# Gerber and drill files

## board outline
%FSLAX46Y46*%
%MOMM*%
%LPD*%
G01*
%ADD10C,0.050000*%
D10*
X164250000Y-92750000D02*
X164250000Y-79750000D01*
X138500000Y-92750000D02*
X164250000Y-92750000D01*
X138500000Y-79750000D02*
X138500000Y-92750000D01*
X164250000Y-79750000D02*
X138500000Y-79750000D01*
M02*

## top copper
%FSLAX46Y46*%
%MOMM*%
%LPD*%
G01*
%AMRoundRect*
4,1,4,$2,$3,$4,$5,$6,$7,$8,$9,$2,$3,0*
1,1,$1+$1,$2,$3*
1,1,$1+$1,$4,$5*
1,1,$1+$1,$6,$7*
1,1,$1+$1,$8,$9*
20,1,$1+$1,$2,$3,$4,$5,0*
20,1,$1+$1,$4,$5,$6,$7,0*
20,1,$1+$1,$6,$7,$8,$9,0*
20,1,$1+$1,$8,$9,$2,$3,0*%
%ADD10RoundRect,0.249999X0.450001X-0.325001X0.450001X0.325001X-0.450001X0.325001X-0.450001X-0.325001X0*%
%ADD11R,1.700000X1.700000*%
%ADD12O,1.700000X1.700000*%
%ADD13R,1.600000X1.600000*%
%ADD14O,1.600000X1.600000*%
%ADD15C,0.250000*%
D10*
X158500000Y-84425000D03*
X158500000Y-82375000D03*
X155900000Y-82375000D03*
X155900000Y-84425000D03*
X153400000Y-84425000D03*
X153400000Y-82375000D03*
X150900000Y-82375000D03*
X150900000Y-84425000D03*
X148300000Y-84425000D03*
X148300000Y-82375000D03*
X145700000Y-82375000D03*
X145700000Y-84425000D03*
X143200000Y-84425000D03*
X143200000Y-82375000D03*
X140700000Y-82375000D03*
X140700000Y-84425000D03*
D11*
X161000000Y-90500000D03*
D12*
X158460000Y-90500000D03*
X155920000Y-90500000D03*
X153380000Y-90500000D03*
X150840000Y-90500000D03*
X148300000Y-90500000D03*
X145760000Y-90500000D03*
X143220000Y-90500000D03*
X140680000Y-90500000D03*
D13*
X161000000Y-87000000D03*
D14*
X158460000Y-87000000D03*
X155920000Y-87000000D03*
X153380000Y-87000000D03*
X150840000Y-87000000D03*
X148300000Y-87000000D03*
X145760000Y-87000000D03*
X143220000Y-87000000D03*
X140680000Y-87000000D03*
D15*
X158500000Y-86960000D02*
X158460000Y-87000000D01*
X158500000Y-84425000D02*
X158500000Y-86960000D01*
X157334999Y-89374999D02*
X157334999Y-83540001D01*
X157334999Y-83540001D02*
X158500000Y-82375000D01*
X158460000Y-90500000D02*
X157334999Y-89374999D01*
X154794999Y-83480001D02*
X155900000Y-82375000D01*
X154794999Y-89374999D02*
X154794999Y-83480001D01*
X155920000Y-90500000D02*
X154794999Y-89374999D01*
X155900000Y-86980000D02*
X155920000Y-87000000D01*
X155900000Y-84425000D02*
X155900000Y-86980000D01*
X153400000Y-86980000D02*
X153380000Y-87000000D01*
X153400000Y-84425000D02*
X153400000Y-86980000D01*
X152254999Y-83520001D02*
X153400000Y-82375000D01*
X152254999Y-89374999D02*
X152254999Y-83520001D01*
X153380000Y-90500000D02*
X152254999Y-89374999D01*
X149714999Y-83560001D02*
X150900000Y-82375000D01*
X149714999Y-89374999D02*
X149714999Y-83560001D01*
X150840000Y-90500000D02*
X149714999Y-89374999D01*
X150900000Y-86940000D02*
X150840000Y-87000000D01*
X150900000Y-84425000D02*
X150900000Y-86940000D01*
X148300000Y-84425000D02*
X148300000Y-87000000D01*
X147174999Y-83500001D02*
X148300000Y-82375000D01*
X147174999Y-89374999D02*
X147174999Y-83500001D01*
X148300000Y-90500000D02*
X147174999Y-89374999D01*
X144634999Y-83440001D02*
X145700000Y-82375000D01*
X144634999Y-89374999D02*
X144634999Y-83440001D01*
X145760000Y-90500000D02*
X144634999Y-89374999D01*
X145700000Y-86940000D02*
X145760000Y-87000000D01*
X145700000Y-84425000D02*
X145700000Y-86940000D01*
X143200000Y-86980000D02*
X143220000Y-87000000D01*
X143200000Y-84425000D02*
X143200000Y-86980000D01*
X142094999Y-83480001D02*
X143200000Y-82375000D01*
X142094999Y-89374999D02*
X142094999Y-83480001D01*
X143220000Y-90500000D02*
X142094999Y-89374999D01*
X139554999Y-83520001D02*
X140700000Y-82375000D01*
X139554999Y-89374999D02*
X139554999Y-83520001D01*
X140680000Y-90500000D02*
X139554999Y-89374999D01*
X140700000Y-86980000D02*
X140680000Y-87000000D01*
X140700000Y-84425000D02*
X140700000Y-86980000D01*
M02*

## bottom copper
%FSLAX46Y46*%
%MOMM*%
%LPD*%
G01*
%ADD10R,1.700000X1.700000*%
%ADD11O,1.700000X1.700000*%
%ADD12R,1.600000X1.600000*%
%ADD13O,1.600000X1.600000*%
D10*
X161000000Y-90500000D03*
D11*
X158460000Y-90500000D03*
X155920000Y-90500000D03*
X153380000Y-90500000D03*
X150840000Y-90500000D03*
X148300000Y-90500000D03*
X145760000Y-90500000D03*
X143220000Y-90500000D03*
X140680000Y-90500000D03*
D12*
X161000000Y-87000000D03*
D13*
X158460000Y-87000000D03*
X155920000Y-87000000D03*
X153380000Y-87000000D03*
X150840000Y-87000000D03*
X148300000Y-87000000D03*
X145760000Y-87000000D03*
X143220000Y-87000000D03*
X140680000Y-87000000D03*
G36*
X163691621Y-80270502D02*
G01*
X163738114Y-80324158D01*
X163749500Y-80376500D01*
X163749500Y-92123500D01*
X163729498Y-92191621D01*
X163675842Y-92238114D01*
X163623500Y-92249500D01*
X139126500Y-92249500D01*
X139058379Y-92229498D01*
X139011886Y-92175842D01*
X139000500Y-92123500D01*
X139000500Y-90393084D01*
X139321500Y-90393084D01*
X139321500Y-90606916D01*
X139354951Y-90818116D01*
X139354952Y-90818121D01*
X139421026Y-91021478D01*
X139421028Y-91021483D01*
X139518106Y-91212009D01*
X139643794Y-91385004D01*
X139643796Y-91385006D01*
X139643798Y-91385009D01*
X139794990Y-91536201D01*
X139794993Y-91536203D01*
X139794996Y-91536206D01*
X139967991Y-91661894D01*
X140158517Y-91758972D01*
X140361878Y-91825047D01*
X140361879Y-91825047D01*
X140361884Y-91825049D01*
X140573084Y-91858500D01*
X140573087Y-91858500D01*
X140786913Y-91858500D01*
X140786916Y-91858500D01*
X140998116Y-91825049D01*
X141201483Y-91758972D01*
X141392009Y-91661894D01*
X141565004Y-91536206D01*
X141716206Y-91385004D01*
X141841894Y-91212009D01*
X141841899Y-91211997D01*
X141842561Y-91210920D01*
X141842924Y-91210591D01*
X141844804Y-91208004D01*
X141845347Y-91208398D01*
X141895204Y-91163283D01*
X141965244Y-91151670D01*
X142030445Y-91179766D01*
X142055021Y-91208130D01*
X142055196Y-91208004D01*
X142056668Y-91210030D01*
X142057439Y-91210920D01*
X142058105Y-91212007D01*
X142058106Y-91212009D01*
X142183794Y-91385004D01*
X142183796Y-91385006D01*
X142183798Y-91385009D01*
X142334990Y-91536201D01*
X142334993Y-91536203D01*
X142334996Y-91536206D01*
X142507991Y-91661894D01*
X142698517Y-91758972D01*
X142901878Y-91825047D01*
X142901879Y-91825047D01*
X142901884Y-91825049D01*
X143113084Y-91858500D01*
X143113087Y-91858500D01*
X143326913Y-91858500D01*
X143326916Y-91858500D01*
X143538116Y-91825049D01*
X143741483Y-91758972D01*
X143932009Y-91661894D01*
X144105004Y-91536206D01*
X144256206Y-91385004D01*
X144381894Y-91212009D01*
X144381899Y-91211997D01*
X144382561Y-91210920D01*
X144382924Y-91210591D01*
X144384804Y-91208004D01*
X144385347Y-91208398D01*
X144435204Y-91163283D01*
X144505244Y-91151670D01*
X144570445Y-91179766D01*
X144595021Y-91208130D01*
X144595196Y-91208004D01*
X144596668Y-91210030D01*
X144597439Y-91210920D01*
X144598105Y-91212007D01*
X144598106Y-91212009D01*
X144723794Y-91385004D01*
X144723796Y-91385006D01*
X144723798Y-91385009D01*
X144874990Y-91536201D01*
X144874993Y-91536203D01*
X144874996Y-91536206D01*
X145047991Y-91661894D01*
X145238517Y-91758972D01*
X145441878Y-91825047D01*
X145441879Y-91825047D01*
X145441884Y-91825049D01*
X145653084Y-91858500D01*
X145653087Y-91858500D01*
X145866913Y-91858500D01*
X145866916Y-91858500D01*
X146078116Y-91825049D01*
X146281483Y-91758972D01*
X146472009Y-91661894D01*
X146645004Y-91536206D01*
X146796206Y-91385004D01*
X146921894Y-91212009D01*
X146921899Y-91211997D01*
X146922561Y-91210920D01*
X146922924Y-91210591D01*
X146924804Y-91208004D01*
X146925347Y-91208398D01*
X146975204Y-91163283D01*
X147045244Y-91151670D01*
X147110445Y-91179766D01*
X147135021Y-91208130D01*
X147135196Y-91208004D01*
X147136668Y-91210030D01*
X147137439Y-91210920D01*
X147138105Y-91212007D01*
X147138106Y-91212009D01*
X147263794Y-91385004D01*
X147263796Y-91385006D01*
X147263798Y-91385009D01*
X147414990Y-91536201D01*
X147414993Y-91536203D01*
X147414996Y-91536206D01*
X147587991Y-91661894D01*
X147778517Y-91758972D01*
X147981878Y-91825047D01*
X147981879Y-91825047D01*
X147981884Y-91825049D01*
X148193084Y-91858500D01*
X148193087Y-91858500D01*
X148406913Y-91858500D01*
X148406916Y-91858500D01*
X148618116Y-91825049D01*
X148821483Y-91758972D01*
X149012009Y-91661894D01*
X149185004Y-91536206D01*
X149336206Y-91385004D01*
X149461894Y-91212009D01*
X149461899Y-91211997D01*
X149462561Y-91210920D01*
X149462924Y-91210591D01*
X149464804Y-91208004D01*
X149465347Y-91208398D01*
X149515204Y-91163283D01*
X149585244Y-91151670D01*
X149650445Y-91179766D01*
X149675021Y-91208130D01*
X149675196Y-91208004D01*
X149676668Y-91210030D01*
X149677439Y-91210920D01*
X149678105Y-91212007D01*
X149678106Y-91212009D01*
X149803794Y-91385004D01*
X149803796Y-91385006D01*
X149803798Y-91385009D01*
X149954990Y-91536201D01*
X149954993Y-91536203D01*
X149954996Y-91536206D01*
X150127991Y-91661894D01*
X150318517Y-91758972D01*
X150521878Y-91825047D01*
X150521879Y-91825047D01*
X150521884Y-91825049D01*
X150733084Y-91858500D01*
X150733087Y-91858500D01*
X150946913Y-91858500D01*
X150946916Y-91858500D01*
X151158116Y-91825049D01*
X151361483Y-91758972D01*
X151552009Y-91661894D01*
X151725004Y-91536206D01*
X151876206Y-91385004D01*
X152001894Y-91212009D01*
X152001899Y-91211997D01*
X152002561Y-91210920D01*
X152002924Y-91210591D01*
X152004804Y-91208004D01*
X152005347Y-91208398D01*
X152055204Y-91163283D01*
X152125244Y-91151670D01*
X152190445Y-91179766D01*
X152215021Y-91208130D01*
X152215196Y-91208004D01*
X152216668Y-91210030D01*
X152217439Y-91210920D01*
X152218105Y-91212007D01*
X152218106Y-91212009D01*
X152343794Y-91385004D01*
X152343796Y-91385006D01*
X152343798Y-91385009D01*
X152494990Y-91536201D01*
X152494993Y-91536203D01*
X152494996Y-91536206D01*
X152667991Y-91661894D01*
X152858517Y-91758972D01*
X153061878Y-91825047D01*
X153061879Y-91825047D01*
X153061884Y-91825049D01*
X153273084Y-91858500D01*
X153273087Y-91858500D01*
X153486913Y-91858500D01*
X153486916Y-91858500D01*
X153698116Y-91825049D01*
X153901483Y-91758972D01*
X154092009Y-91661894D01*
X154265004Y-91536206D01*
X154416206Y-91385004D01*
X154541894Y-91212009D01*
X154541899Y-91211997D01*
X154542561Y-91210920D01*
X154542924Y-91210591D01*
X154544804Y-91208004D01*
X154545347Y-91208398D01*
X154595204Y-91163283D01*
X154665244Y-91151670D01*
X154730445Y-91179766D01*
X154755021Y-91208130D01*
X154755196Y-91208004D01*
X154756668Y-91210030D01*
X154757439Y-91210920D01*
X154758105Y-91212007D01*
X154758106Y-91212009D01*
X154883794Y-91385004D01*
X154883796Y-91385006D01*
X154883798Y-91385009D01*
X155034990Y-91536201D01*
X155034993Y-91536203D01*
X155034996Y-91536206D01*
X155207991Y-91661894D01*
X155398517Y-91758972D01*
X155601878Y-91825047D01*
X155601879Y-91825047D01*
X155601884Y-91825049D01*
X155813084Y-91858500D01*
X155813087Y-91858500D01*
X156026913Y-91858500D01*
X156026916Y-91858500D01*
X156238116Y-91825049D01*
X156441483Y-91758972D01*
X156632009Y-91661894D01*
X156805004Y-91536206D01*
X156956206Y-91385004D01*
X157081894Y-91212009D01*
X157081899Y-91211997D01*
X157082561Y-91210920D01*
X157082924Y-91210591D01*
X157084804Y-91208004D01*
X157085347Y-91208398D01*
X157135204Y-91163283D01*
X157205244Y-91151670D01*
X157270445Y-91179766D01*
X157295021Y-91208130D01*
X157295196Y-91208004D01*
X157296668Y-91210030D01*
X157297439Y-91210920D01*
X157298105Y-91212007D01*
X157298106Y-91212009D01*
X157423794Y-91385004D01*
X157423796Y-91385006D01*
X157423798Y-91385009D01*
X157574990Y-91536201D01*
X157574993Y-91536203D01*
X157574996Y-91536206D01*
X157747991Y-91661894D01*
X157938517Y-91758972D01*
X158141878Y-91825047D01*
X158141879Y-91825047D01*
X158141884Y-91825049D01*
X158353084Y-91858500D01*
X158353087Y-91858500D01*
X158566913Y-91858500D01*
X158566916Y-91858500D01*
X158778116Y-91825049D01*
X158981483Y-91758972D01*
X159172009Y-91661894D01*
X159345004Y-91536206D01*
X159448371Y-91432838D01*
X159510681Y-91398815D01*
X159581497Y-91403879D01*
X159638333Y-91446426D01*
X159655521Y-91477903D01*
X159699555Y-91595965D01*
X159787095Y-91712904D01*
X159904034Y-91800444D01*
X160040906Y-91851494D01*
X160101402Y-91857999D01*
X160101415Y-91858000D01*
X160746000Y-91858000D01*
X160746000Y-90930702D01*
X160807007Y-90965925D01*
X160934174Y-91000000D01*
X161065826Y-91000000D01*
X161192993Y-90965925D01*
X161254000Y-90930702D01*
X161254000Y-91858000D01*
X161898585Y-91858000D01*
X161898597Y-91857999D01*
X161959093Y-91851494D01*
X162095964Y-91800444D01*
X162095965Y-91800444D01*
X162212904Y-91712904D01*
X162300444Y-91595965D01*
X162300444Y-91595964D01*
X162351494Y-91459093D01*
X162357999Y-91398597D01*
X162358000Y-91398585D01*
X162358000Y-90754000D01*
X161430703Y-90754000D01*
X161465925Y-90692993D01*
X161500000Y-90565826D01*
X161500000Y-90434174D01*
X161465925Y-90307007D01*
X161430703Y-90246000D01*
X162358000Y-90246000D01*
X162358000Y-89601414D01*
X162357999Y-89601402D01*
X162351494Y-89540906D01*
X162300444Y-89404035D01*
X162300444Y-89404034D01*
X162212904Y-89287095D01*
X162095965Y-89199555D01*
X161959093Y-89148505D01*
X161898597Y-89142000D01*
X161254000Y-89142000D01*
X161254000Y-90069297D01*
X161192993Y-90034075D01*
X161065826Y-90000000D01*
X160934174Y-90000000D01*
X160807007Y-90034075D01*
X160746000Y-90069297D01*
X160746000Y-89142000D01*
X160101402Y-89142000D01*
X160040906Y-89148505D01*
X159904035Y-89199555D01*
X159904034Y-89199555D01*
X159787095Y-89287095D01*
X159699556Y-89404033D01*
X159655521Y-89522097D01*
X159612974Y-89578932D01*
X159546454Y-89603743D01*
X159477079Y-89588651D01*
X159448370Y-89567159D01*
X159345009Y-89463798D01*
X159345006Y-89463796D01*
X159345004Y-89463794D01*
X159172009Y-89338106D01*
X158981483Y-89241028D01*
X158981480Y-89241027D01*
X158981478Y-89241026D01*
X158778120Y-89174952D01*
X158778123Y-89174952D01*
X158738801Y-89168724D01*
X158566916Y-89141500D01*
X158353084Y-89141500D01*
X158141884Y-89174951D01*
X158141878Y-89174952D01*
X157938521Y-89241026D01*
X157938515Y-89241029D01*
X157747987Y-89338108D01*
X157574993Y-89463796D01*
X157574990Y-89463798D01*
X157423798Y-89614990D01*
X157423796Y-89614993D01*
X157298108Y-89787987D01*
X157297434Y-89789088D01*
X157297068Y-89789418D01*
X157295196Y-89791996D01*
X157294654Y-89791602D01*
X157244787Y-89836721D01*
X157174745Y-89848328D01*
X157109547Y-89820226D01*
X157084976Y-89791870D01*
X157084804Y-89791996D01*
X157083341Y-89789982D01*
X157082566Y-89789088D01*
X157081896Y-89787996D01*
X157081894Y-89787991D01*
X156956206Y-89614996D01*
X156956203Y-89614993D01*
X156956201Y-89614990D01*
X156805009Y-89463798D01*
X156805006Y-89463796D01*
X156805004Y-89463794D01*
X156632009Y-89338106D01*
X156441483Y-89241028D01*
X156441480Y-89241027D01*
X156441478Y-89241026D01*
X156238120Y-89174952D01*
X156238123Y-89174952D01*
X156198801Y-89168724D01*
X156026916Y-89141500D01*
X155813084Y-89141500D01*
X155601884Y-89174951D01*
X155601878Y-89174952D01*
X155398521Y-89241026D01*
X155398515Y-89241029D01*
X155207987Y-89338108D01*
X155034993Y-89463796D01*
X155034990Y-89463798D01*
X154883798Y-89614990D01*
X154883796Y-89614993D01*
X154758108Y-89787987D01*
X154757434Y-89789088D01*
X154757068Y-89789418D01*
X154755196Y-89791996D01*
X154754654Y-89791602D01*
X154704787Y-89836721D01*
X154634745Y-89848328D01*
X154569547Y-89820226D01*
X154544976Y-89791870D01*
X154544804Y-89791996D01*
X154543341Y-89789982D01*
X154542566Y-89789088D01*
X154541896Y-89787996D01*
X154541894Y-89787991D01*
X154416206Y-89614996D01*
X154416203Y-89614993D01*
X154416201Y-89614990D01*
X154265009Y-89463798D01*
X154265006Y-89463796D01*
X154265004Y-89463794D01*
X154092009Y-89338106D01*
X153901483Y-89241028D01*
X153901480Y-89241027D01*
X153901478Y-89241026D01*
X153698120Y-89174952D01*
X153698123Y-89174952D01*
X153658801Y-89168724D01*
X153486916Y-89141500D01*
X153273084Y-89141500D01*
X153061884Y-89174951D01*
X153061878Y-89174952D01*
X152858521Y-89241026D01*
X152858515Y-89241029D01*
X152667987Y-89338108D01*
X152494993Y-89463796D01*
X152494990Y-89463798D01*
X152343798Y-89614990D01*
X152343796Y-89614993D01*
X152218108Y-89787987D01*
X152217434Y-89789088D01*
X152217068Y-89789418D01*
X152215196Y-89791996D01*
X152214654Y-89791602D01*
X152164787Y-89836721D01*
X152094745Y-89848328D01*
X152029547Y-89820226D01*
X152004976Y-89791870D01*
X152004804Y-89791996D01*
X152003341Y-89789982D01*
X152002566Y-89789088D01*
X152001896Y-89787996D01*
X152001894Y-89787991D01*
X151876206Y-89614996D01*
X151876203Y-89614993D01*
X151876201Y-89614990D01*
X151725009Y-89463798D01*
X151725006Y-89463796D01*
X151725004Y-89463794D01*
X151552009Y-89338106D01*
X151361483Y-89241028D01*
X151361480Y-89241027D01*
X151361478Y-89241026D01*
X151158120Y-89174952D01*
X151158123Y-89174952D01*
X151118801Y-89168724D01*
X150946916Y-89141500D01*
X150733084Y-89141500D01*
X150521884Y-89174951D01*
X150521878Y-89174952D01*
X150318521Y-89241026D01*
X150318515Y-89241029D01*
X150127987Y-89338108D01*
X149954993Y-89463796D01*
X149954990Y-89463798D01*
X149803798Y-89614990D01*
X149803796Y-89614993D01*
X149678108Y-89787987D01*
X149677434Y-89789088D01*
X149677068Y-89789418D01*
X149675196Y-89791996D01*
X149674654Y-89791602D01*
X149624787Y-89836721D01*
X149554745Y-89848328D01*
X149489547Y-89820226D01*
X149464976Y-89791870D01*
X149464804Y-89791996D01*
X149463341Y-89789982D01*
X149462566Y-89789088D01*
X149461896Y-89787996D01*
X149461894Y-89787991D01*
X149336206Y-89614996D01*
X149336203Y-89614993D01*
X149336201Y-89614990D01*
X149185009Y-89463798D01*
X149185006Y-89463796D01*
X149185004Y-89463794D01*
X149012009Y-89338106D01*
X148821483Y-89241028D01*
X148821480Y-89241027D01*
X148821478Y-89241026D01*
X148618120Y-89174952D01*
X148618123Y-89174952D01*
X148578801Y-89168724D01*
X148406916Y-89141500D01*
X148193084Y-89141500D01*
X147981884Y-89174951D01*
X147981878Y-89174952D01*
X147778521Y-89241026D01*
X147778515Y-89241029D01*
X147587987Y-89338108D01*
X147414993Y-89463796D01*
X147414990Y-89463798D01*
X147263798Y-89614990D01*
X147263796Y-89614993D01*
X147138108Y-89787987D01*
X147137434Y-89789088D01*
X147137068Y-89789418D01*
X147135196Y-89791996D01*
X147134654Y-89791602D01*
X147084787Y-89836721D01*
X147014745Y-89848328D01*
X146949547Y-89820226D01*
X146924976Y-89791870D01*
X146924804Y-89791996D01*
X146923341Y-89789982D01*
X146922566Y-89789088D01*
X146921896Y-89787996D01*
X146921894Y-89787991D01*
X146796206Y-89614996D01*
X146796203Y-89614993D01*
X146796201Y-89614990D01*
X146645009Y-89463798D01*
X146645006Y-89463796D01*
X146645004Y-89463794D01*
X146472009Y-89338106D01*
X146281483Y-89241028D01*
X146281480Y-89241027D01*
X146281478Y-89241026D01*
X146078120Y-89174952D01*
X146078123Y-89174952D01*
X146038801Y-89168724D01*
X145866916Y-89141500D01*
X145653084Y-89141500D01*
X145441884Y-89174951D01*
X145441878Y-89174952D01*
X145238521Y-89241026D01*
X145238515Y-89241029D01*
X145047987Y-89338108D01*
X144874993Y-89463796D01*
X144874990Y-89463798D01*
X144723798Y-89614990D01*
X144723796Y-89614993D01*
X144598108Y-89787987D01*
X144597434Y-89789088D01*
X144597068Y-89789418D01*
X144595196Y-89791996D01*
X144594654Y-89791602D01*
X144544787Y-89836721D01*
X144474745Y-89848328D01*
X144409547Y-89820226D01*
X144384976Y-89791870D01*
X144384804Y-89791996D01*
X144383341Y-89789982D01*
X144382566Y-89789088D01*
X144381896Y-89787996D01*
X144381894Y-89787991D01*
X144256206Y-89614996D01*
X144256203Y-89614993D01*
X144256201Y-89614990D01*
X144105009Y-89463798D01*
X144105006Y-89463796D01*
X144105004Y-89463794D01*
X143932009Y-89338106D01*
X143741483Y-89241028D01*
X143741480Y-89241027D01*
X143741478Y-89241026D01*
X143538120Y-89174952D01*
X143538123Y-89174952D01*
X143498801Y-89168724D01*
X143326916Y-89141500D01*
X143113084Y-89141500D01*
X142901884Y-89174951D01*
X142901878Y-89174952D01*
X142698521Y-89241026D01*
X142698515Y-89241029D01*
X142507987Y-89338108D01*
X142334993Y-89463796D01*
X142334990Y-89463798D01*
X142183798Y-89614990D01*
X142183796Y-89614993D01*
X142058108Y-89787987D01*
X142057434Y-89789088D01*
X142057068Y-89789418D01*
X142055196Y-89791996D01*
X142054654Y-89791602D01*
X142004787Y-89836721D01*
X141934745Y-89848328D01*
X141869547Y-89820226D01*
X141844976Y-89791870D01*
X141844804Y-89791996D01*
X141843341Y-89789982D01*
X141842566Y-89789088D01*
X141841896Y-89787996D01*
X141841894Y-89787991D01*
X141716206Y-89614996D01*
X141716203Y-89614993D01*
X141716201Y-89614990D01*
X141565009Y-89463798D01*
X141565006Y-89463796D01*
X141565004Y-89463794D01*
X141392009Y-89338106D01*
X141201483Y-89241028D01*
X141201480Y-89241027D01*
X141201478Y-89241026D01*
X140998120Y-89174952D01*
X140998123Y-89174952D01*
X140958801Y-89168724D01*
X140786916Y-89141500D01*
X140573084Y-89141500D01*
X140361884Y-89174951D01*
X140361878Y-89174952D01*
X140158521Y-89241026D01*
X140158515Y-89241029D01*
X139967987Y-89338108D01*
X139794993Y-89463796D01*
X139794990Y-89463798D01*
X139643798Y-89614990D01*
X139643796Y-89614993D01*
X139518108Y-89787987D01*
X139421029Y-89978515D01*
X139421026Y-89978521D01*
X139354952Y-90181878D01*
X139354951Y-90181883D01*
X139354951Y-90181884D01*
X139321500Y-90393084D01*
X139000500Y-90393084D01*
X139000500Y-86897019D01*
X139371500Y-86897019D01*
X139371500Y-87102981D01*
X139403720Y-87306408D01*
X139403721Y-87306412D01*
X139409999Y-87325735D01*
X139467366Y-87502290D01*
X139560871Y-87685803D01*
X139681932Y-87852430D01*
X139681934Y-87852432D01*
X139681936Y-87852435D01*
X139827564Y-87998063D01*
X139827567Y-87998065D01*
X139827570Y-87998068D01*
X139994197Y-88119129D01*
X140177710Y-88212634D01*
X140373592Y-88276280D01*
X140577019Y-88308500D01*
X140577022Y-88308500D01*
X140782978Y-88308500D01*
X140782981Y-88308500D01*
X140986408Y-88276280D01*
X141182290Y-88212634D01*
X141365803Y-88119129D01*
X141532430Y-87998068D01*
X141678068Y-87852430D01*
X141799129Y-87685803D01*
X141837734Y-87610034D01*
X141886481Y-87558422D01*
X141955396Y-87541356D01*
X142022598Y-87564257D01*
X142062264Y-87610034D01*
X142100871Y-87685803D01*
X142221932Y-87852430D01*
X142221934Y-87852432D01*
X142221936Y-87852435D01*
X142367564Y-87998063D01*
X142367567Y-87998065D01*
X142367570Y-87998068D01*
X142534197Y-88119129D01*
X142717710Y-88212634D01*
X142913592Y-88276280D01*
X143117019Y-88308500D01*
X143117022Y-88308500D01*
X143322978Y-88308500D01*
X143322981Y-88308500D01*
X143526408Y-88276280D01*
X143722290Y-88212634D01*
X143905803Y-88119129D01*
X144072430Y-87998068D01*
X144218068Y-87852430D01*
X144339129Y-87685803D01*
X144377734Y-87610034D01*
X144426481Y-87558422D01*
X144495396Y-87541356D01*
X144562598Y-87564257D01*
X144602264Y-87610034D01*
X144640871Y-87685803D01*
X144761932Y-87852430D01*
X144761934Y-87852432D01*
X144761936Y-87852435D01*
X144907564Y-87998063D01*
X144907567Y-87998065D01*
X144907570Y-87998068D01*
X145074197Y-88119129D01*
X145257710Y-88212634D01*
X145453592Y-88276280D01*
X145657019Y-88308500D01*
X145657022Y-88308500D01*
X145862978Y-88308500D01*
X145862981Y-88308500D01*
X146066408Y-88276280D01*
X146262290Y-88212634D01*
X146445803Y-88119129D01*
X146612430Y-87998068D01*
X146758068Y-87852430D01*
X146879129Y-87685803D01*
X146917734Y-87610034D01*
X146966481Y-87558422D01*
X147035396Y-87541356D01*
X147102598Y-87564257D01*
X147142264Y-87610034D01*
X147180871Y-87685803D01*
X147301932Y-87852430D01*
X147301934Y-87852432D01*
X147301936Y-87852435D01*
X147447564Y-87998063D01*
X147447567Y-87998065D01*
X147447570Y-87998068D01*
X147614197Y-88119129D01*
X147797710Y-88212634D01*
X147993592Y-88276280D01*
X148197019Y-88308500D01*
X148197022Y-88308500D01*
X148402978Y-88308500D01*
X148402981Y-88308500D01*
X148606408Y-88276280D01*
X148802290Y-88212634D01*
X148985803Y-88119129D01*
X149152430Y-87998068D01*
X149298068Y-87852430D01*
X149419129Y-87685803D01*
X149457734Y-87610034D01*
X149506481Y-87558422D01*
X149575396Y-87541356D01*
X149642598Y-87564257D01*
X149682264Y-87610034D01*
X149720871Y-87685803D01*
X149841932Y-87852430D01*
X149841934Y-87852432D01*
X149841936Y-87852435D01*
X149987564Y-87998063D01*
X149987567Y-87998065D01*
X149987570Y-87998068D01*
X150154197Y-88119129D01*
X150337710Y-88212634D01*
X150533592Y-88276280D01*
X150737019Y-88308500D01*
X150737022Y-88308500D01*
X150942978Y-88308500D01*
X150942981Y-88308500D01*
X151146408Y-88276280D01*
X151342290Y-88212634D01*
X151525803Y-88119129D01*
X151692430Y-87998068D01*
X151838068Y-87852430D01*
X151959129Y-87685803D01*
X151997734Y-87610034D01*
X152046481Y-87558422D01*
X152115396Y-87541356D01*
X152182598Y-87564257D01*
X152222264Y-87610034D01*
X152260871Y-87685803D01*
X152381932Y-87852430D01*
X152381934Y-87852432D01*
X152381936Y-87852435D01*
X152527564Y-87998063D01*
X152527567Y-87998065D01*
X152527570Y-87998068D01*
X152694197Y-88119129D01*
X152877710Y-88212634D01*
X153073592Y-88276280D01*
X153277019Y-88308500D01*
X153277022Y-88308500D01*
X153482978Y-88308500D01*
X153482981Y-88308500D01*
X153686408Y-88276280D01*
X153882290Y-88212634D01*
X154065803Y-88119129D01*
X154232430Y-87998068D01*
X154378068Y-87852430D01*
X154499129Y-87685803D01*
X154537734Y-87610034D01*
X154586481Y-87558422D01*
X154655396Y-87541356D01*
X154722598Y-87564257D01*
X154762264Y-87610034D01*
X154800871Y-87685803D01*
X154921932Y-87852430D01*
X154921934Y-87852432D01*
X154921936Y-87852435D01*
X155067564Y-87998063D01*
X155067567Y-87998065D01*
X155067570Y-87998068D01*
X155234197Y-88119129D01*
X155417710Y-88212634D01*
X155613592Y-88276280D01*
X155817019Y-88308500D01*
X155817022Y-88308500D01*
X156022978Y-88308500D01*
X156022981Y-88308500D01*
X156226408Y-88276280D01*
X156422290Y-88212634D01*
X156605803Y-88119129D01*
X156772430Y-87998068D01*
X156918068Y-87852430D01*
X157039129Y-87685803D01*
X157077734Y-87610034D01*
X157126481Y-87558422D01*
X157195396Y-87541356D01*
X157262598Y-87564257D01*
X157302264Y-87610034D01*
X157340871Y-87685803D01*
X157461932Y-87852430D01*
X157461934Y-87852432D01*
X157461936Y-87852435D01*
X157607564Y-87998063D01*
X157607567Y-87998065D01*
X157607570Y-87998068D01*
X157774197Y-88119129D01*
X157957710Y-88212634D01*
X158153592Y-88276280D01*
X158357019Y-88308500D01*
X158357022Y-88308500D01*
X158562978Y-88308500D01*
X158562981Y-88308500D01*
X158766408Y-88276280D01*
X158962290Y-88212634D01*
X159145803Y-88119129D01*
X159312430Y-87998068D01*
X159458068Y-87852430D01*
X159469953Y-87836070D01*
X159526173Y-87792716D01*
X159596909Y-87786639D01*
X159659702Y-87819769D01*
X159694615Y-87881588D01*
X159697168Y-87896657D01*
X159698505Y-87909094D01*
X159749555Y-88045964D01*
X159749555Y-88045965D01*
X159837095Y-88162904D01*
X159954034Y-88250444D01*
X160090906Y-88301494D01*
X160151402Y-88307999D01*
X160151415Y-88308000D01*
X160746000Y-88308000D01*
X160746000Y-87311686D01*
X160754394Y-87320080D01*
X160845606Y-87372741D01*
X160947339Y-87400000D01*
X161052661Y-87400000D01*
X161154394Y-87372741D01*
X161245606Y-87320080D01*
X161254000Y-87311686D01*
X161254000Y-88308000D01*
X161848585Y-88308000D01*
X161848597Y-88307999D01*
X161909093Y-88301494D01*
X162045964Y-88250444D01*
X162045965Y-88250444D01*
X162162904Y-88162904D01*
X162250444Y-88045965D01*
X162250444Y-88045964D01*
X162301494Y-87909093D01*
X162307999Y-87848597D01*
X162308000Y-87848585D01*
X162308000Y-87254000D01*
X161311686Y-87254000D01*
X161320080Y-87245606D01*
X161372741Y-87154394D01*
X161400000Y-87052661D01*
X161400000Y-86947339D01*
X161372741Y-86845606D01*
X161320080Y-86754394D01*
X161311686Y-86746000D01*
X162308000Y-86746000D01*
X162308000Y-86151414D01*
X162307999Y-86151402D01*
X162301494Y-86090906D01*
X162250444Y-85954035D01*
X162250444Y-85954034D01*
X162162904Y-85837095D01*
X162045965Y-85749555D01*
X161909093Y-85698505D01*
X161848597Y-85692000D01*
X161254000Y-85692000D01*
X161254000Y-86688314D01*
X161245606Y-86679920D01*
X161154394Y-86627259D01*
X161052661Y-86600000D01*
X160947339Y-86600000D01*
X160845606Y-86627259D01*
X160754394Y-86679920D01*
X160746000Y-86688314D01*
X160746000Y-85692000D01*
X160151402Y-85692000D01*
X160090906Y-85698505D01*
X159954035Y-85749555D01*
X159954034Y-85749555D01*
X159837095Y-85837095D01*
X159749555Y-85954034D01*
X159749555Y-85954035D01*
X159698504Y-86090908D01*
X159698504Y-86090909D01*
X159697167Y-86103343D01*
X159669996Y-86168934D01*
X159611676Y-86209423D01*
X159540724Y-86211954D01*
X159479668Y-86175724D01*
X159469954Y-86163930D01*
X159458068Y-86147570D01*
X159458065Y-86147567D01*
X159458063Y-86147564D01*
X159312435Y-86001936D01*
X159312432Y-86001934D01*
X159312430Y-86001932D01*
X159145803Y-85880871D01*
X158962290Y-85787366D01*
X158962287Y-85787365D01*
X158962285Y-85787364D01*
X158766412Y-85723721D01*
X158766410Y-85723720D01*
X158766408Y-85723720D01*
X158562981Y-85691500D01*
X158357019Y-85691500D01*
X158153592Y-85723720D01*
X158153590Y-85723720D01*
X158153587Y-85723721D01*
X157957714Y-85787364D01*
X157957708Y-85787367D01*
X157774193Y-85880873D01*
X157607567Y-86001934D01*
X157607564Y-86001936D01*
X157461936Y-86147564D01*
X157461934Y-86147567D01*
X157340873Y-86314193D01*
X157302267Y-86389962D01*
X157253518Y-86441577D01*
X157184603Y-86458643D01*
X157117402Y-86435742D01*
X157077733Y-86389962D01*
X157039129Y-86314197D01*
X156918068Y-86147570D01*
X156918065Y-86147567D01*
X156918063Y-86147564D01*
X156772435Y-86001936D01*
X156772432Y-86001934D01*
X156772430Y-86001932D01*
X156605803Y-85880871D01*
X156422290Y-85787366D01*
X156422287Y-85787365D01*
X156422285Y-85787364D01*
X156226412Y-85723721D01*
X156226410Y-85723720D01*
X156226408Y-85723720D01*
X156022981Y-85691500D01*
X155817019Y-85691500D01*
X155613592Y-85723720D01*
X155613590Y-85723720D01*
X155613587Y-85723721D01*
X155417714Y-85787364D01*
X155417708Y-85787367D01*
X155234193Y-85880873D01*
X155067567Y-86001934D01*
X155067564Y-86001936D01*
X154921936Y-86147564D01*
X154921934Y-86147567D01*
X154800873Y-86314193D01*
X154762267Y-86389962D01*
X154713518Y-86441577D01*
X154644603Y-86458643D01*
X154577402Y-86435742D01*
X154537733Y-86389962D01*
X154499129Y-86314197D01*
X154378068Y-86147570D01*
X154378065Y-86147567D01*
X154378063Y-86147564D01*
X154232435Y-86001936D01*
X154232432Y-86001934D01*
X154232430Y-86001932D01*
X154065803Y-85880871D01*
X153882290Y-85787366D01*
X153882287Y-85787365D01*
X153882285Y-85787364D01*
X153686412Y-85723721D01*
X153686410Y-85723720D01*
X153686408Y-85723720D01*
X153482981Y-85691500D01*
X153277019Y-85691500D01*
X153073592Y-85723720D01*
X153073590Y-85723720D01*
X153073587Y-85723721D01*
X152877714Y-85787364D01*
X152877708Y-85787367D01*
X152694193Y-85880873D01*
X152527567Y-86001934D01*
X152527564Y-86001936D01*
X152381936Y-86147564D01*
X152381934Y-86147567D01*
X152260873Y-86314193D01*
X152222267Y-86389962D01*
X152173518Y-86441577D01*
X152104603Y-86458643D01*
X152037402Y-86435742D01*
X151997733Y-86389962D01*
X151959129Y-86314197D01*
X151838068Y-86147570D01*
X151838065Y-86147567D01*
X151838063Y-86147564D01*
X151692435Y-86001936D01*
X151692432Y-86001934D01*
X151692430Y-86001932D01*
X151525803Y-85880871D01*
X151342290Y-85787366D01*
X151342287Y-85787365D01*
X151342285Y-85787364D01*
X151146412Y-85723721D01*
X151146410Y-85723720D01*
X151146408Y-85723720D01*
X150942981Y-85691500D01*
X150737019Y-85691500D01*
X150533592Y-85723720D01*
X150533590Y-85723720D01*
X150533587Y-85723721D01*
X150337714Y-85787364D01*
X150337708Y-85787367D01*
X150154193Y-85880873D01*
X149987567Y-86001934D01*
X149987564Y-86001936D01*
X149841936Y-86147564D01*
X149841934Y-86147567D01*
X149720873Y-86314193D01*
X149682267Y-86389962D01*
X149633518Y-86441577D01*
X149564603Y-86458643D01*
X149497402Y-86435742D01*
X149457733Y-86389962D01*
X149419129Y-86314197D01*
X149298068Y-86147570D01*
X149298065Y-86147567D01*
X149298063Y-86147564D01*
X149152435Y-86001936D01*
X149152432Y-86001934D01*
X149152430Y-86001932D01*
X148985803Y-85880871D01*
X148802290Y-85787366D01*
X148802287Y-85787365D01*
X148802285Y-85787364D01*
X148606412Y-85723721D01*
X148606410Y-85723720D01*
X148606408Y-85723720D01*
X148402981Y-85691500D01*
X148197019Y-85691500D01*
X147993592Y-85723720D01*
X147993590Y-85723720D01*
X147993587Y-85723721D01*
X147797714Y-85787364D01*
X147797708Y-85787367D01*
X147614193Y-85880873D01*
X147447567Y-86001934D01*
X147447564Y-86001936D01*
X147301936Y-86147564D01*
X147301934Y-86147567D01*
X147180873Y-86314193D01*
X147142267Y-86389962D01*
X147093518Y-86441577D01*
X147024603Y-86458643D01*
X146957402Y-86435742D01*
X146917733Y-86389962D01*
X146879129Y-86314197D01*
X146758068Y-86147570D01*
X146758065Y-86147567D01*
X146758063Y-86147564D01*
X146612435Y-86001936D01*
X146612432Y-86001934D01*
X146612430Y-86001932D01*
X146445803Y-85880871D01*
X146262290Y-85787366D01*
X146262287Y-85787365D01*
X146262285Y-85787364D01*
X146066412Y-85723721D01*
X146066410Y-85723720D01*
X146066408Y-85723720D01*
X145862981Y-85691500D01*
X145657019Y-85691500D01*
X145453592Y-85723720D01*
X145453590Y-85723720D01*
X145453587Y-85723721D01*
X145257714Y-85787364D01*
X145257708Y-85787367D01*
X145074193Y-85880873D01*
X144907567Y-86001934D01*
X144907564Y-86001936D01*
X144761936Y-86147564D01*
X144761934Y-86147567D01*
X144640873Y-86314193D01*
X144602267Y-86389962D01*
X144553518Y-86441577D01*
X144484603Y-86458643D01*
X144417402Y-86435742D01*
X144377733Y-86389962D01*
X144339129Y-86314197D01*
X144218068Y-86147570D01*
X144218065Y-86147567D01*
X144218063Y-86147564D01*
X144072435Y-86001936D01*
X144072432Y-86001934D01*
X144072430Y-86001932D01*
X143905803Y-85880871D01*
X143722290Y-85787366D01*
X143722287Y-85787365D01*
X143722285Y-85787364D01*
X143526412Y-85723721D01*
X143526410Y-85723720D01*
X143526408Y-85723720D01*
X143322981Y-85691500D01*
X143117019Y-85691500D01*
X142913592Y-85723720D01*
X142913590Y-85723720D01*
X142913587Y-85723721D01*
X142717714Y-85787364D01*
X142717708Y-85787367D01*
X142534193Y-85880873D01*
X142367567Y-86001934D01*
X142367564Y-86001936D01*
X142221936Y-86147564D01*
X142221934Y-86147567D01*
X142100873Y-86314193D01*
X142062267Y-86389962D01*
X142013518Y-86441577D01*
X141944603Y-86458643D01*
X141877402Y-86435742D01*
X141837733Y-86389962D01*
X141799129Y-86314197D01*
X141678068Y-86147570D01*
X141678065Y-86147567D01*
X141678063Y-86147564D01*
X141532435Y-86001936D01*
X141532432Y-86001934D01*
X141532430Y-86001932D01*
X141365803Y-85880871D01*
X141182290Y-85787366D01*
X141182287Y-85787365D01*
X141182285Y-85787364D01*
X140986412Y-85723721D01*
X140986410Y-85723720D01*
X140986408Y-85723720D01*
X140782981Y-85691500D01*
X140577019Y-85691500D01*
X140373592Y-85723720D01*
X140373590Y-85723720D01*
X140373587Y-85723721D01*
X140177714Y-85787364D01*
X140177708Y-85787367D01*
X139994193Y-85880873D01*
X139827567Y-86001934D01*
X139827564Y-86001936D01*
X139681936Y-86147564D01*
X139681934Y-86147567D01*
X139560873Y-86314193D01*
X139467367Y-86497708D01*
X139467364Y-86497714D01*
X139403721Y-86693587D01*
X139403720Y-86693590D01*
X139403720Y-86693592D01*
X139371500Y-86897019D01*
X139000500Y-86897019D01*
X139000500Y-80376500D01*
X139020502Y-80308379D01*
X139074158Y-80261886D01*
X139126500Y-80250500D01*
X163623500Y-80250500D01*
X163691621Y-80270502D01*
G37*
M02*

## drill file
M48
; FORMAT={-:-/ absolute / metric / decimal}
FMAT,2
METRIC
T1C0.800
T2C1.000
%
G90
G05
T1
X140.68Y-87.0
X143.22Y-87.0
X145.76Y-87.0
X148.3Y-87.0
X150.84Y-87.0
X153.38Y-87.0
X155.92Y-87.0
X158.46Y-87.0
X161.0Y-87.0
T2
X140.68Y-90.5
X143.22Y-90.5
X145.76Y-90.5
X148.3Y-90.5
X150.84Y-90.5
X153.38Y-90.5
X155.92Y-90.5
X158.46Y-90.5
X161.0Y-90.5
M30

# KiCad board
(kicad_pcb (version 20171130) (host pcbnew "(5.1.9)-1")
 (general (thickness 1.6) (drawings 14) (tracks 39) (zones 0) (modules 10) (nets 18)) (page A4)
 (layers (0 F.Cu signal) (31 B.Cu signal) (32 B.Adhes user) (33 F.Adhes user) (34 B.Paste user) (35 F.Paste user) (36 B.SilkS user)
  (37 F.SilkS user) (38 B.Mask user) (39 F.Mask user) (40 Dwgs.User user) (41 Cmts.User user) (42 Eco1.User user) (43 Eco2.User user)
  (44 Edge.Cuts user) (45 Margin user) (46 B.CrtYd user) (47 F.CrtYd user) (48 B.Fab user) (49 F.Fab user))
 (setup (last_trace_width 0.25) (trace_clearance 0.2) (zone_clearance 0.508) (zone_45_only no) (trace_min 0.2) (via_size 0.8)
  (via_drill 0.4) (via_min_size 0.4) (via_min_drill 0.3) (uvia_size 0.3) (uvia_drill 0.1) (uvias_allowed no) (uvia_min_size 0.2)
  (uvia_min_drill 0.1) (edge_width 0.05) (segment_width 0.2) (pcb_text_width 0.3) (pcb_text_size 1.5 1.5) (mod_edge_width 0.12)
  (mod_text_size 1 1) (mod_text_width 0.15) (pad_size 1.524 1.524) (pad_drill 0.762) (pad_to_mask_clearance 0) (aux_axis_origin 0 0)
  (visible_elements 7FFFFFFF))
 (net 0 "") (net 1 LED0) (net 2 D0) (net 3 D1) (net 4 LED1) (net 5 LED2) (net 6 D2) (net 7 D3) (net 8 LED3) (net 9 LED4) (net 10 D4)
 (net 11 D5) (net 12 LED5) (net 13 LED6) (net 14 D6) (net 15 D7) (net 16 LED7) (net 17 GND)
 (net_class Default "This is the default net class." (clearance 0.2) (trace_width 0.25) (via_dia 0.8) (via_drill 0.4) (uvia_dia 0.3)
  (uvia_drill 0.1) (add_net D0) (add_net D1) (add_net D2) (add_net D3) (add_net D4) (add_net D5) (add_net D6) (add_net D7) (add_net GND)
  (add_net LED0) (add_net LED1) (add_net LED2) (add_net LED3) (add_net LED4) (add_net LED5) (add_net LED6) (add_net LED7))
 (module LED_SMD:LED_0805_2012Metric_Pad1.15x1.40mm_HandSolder (layer F.Cu) (at 158.5 83.4 90)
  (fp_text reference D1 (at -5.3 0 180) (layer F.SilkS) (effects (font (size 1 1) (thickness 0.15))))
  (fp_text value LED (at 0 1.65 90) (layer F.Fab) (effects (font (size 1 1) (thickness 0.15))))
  (pad 1 smd roundrect (at -1.025 0 90) (size 1.15 1.4) (layers F.Cu F.Paste F.Mask) (roundrect_rratio 0.2173904347826087) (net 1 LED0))
  (pad 2 smd roundrect (at 1.025 0 90) (size 1.15 1.4) (layers F.Cu F.Paste F.Mask) (roundrect_rratio 0.2173904347826087) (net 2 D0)))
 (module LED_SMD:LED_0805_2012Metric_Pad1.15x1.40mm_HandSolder (layer F.Cu) (at 155.9 83.4 90)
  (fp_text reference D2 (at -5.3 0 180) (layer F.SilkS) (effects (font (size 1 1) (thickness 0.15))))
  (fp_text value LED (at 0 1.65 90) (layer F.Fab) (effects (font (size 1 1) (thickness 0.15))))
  (pad 2 smd roundrect (at 1.025 0 90) (size 1.15 1.4) (layers F.Cu F.Paste F.Mask) (roundrect_rratio 0.2173904347826087) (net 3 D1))
  (pad 1 smd roundrect (at -1.025 0 90) (size 1.15 1.4) (layers F.Cu F.Paste F.Mask) (roundrect_rratio 0.2173904347826087) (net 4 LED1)))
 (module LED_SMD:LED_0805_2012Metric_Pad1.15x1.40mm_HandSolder (layer F.Cu) (at 153.4 83.4 90)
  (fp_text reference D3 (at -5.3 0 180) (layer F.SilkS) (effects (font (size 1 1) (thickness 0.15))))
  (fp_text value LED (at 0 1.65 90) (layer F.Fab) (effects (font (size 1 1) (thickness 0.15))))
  (pad 1 smd roundrect (at -1.025 0 90) (size 1.15 1.4) (layers F.Cu F.Paste F.Mask) (roundrect_rratio 0.2173904347826087) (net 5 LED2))
  (pad 2 smd roundrect (at 1.025 0 90) (size 1.15 1.4) (layers F.Cu F.Paste F.Mask) (roundrect_rratio 0.2173904347826087) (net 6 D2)))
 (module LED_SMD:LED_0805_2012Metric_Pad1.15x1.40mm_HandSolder (layer F.Cu) (at 150.9 83.4 90)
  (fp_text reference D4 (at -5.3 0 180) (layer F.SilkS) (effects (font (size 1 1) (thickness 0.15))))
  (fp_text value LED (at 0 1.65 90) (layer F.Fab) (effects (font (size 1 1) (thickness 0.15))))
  (pad 2 smd roundrect (at 1.025 0 90) (size 1.15 1.4) (layers F.Cu F.Paste F.Mask) (roundrect_rratio 0.2173904347826087) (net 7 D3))
  (pad 1 smd roundrect (at -1.025 0 90) (size 1.15 1.4) (layers F.Cu F.Paste F.Mask) (roundrect_rratio 0.2173904347826087) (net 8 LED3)))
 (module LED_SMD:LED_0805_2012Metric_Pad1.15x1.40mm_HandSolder (layer F.Cu) (at 148.3 83.4 90)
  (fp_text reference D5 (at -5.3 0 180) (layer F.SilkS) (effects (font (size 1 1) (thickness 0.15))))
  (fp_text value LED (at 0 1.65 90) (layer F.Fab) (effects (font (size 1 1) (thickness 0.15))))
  (pad 1 smd roundrect (at -1.025 0 90) (size 1.15 1.4) (layers F.Cu F.Paste F.Mask) (roundrect_rratio 0.2173904347826087) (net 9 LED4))
  (pad 2 smd roundrect (at 1.025 0 90) (size 1.15 1.4) (layers F.Cu F.Paste F.Mask) (roundrect_rratio 0.2173904347826087) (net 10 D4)))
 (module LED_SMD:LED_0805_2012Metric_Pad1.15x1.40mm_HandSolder (layer F.Cu) (at 145.7 83.4 90)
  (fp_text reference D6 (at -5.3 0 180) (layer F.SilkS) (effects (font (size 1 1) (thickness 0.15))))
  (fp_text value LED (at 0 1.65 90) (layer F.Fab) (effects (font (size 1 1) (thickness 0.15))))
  (pad 2 smd roundrect (at 1.025 0 90) (size 1.15 1.4) (layers F.Cu F.Paste F.Mask) (roundrect_rratio 0.2173904347826087) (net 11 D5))
  (pad 1 smd roundrect (at -1.025 0 90) (size 1.15 1.4) (layers F.Cu F.Paste F.Mask) (roundrect_rratio 0.2173904347826087) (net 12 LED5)))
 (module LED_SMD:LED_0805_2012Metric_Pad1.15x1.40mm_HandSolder (layer F.Cu) (at 143.2 83.4 90)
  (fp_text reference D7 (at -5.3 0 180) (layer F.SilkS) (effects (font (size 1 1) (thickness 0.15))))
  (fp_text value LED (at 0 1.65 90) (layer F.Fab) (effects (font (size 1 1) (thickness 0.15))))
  (pad 1 smd roundrect (at -1.025 0 90) (size 1.15 1.4) (layers F.Cu F.Paste F.Mask) (roundrect_rratio 0.2173904347826087) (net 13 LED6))
  (pad 2 smd roundrect (at 1.025 0 90) (size 1.15 1.4) (layers F.Cu F.Paste F.Mask) (roundrect_rratio 0.2173904347826087) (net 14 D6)))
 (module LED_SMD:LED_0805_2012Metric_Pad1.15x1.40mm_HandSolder (layer F.Cu) (at 140.7 83.4 90)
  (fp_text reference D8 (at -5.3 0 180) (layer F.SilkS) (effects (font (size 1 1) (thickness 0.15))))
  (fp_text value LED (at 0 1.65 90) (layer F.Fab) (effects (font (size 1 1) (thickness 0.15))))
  (pad 2 smd roundrect (at 1.025 0 90) (size 1.15 1.4) (layers F.Cu F.Paste F.Mask) (roundrect_rratio 0.2173904347826087) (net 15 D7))
  (pad 1 smd roundrect (at -1.025 0 90) (size 1.15 1.4) (layers F.Cu F.Paste F.Mask) (roundrect_rratio 0.2173904347826087) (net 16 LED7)))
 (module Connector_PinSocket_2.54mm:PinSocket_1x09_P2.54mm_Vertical (layer F.Cu) (at 161 90.5 270)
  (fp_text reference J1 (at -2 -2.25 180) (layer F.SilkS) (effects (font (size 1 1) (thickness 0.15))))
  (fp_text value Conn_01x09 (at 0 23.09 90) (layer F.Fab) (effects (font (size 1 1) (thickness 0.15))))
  (pad 1 thru_hole rect (at 0 0 270) (size 1.7 1.7) (drill 1) (layers *.Cu *.Mask) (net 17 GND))
  (pad 2 thru_hole oval (at 0 2.54 270) (size 1.7 1.7) (drill 1) (layers *.Cu *.Mask) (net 2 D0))
  (pad 3 thru_hole oval (at 0 5.08 270) (size 1.7 1.7) (drill 1) (layers *.Cu *.Mask) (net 3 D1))
  (pad 4 thru_hole oval (at 0 7.62 270) (size 1.7 1.7) (drill 1) (layers *.Cu *.Mask) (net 6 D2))
  (pad 5 thru_hole oval (at 0 10.16 270) (size 1.7 1.7) (drill 1) (layers *.Cu *.Mask) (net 7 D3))
  (pad 6 thru_hole oval (at 0 12.7 270) (size 1.7 1.7) (drill 1) (layers *.Cu *.Mask) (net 10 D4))
  (pad 7 thru_hole oval (at 0 15.24 270) (size 1.7 1.7) (drill 1) (layers *.Cu *.Mask) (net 11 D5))
  (pad 8 thru_hole oval (at 0 17.78 270) (size 1.7 1.7) (drill 1) (layers *.Cu *.Mask) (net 14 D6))
  (pad 9 thru_hole oval (at 0 20.32 270) (size 1.7 1.7) (drill 1) (layers *.Cu *.Mask) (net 15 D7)))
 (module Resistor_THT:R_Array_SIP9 (layer F.Cu) (at 161 87 180)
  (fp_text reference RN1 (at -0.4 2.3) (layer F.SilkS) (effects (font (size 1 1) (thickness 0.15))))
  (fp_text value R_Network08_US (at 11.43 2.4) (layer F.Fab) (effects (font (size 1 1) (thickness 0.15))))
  (pad 1 thru_hole rect (at 0 0 180) (size 1.6 1.6) (drill 0.8) (layers *.Cu *.Mask) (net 17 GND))
  (pad 2 thru_hole oval (at 2.54 0 180) (size 1.6 1.6) (drill 0.8) (layers *.Cu *.Mask) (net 1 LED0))
  (pad 3 thru_hole oval (at 5.08 0 180) (size 1.6 1.6) (drill 0.8) (layers *.Cu *.Mask) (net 4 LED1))
  (pad 4 thru_hole oval (at 7.62 0 180) (size 1.6 1.6) (drill 0.8) (layers *.Cu *.Mask) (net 5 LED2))
  (pad 5 thru_hole oval (at 10.16 0 180) (size 1.6 1.6) (drill 0.8) (layers *.Cu *.Mask) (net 8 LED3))
  (pad 6 thru_hole oval (at 12.7 0 180) (size 1.6 1.6) (drill 0.8) (layers *.Cu *.Mask) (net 9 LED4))
  (pad 7 thru_hole oval (at 15.24 0 180) (size 1.6 1.6) (drill 0.8) (layers *.Cu *.Mask) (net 12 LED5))
  (pad 8 thru_hole oval (at 17.78 0 180) (size 1.6 1.6) (drill 0.8) (layers *.Cu *.Mask) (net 13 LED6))
  (pad 9 thru_hole oval (at 20.32 0 180) (size 1.6 1.6) (drill 0.8) (layers *.Cu *.Mask) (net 16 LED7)))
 (gr_line (start 164.25 92.75) (end 164.25 79.75) (layer Edge.Cuts) (width 0.05))
 (gr_line (start 138.5 92.75) (end 164.25 92.75) (layer Edge.Cuts) (width 0.05))
 (gr_line (start 138.5 79.75) (end 138.5 92.75) (layer Edge.Cuts) (width 0.05))
 (gr_line (start 164.25 79.75) (end 138.5 79.75) (layer Edge.Cuts) (width 0.05))
 (segment (start 158.5 86.96) (end 158.46 87) (width 0.25) (layer F.Cu) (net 1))
 (segment (start 158.5 84.425) (end 158.5 86.96) (width 0.25) (layer F.Cu) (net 1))
 (segment (start 157.334999 89.374999) (end 157.334999 83.540001) (width 0.25) (layer F.Cu) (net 2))
 (segment (start 157.334999 83.540001) (end 158.5 82.375) (width 0.25) (layer F.Cu) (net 2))
 (segment (start 158.46 90.5) (end 157.334999 89.374999) (width 0.25) (layer F.Cu) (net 2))
 (segment (start 154.794999 83.480001) (end 155.9 82.375) (width 0.25) (layer F.Cu) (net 3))
 (segment (start 154.794999 89.374999) (end 154.794999 83.480001) (width 0.25) (layer F.Cu) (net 3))
 (segment (start 155.92 90.5) (end 154.794999 89.374999) (width 0.25) (layer F.Cu) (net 3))
 (segment (start 155.9 86.98) (end 155.92 87) (width 0.25) (layer F.Cu) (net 4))
 (segment (start 155.9 84.425) (end 155.9 86.98) (width 0.25) (layer F.Cu) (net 4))
 (segment (start 153.4 86.98) (end 153.38 87) (width 0.25) (layer F.Cu) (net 5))
 (segment (start 153.4 84.425) (end 153.4 86.98) (width 0.25) (layer F.Cu) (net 5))
 (segment (start 152.254999 83.520001) (end 153.4 82.375) (width 0.25) (layer F.Cu) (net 6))
 (segment (start 152.254999 89.374999) (end 152.254999 83.520001) (width 0.25) (layer F.Cu) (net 6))
 (segment (start 153.38 90.5) (end 152.254999 89.374999) (width 0.25) (layer F.Cu) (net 6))
 (segment (start 149.714999 83.560001) (end 150.9 82.375) (width 0.25) (layer F.Cu) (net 7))
 (segment (start 149.714999 89.374999) (end 149.714999 83.560001) (width 0.25) (layer F.Cu) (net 7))
 (segment (start 150.84 90.5) (end 149.714999 89.374999) (width 0.25) (layer F.Cu) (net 7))
 (segment (start 150.9 86.94) (end 150.84 87) (width 0.25) (layer F.Cu) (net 8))
 (segment (start 150.9 84.425) (end 150.9 86.94) (width 0.25) (layer F.Cu) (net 8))
 (segment (start 148.3 84.425) (end 148.3 87) (width 0.25) (layer F.Cu) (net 9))
 (segment (start 147.174999 83.500001) (end 148.3 82.375) (width 0.25) (layer F.Cu) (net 10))
 (segment (start 147.174999 89.374999) (end 147.174999 83.500001) (width 0.25) (layer F.Cu) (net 10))
 (segment (start 148.3 90.5) (end 147.174999 89.374999) (width 0.25) (layer F.Cu) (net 10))
 (segment (start 144.634999 83.440001) (end 145.7 82.375) (width 0.25) (layer F.Cu) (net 11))
 (segment (start 144.634999 89.374999) (end 144.634999 83.440001) (width 0.25) (layer F.Cu) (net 11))
 (segment (start 145.76 90.5) (end 144.634999 89.374999) (width 0.25) (layer F.Cu) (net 11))
 (segment (start 145.7 86.94) (end 145.76 87) (width 0.25) (layer F.Cu) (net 12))
 (segment (start 145.7 84.425) (end 145.7 86.94) (width 0.25) (layer F.Cu) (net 12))
 (segment (start 143.2 86.98) (end 143.22 87) (width 0.25) (layer F.Cu) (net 13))
 (segment (start 143.2 84.425) (end 143.2 86.98) (width 0.25) (layer F.Cu) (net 13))
 (segment (start 142.094999 83.480001) (end 143.2 82.375) (width 0.25) (layer F.Cu) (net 14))
 (segment (start 142.094999 89.374999) (end 142.094999 83.480001) (width 0.25) (layer F.Cu) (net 14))
 (segment (start 143.22 90.5) (end 142.094999 89.374999) (width 0.25) (layer F.Cu) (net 14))
 (segment (start 139.554999 83.520001) (end 140.7 82.375) (width 0.25) (layer F.Cu) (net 15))
 (segment (start 139.554999 89.374999) (end 139.554999 83.520001) (width 0.25) (layer F.Cu) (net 15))
 (segment (start 140.68 90.5) (end 139.554999 89.374999) (width 0.25) (layer F.Cu) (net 15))
 (segment (start 140.7 86.98) (end 140.68 87) (width 0.25) (layer F.Cu) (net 16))
 (segment (start 140.7 84.425) (end 140.7 86.98) (width 0.25) (layer F.Cu) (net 16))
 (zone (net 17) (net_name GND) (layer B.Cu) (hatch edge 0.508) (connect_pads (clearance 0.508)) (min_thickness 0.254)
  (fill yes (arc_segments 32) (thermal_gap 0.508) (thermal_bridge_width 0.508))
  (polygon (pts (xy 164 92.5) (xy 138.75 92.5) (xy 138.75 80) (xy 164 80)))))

